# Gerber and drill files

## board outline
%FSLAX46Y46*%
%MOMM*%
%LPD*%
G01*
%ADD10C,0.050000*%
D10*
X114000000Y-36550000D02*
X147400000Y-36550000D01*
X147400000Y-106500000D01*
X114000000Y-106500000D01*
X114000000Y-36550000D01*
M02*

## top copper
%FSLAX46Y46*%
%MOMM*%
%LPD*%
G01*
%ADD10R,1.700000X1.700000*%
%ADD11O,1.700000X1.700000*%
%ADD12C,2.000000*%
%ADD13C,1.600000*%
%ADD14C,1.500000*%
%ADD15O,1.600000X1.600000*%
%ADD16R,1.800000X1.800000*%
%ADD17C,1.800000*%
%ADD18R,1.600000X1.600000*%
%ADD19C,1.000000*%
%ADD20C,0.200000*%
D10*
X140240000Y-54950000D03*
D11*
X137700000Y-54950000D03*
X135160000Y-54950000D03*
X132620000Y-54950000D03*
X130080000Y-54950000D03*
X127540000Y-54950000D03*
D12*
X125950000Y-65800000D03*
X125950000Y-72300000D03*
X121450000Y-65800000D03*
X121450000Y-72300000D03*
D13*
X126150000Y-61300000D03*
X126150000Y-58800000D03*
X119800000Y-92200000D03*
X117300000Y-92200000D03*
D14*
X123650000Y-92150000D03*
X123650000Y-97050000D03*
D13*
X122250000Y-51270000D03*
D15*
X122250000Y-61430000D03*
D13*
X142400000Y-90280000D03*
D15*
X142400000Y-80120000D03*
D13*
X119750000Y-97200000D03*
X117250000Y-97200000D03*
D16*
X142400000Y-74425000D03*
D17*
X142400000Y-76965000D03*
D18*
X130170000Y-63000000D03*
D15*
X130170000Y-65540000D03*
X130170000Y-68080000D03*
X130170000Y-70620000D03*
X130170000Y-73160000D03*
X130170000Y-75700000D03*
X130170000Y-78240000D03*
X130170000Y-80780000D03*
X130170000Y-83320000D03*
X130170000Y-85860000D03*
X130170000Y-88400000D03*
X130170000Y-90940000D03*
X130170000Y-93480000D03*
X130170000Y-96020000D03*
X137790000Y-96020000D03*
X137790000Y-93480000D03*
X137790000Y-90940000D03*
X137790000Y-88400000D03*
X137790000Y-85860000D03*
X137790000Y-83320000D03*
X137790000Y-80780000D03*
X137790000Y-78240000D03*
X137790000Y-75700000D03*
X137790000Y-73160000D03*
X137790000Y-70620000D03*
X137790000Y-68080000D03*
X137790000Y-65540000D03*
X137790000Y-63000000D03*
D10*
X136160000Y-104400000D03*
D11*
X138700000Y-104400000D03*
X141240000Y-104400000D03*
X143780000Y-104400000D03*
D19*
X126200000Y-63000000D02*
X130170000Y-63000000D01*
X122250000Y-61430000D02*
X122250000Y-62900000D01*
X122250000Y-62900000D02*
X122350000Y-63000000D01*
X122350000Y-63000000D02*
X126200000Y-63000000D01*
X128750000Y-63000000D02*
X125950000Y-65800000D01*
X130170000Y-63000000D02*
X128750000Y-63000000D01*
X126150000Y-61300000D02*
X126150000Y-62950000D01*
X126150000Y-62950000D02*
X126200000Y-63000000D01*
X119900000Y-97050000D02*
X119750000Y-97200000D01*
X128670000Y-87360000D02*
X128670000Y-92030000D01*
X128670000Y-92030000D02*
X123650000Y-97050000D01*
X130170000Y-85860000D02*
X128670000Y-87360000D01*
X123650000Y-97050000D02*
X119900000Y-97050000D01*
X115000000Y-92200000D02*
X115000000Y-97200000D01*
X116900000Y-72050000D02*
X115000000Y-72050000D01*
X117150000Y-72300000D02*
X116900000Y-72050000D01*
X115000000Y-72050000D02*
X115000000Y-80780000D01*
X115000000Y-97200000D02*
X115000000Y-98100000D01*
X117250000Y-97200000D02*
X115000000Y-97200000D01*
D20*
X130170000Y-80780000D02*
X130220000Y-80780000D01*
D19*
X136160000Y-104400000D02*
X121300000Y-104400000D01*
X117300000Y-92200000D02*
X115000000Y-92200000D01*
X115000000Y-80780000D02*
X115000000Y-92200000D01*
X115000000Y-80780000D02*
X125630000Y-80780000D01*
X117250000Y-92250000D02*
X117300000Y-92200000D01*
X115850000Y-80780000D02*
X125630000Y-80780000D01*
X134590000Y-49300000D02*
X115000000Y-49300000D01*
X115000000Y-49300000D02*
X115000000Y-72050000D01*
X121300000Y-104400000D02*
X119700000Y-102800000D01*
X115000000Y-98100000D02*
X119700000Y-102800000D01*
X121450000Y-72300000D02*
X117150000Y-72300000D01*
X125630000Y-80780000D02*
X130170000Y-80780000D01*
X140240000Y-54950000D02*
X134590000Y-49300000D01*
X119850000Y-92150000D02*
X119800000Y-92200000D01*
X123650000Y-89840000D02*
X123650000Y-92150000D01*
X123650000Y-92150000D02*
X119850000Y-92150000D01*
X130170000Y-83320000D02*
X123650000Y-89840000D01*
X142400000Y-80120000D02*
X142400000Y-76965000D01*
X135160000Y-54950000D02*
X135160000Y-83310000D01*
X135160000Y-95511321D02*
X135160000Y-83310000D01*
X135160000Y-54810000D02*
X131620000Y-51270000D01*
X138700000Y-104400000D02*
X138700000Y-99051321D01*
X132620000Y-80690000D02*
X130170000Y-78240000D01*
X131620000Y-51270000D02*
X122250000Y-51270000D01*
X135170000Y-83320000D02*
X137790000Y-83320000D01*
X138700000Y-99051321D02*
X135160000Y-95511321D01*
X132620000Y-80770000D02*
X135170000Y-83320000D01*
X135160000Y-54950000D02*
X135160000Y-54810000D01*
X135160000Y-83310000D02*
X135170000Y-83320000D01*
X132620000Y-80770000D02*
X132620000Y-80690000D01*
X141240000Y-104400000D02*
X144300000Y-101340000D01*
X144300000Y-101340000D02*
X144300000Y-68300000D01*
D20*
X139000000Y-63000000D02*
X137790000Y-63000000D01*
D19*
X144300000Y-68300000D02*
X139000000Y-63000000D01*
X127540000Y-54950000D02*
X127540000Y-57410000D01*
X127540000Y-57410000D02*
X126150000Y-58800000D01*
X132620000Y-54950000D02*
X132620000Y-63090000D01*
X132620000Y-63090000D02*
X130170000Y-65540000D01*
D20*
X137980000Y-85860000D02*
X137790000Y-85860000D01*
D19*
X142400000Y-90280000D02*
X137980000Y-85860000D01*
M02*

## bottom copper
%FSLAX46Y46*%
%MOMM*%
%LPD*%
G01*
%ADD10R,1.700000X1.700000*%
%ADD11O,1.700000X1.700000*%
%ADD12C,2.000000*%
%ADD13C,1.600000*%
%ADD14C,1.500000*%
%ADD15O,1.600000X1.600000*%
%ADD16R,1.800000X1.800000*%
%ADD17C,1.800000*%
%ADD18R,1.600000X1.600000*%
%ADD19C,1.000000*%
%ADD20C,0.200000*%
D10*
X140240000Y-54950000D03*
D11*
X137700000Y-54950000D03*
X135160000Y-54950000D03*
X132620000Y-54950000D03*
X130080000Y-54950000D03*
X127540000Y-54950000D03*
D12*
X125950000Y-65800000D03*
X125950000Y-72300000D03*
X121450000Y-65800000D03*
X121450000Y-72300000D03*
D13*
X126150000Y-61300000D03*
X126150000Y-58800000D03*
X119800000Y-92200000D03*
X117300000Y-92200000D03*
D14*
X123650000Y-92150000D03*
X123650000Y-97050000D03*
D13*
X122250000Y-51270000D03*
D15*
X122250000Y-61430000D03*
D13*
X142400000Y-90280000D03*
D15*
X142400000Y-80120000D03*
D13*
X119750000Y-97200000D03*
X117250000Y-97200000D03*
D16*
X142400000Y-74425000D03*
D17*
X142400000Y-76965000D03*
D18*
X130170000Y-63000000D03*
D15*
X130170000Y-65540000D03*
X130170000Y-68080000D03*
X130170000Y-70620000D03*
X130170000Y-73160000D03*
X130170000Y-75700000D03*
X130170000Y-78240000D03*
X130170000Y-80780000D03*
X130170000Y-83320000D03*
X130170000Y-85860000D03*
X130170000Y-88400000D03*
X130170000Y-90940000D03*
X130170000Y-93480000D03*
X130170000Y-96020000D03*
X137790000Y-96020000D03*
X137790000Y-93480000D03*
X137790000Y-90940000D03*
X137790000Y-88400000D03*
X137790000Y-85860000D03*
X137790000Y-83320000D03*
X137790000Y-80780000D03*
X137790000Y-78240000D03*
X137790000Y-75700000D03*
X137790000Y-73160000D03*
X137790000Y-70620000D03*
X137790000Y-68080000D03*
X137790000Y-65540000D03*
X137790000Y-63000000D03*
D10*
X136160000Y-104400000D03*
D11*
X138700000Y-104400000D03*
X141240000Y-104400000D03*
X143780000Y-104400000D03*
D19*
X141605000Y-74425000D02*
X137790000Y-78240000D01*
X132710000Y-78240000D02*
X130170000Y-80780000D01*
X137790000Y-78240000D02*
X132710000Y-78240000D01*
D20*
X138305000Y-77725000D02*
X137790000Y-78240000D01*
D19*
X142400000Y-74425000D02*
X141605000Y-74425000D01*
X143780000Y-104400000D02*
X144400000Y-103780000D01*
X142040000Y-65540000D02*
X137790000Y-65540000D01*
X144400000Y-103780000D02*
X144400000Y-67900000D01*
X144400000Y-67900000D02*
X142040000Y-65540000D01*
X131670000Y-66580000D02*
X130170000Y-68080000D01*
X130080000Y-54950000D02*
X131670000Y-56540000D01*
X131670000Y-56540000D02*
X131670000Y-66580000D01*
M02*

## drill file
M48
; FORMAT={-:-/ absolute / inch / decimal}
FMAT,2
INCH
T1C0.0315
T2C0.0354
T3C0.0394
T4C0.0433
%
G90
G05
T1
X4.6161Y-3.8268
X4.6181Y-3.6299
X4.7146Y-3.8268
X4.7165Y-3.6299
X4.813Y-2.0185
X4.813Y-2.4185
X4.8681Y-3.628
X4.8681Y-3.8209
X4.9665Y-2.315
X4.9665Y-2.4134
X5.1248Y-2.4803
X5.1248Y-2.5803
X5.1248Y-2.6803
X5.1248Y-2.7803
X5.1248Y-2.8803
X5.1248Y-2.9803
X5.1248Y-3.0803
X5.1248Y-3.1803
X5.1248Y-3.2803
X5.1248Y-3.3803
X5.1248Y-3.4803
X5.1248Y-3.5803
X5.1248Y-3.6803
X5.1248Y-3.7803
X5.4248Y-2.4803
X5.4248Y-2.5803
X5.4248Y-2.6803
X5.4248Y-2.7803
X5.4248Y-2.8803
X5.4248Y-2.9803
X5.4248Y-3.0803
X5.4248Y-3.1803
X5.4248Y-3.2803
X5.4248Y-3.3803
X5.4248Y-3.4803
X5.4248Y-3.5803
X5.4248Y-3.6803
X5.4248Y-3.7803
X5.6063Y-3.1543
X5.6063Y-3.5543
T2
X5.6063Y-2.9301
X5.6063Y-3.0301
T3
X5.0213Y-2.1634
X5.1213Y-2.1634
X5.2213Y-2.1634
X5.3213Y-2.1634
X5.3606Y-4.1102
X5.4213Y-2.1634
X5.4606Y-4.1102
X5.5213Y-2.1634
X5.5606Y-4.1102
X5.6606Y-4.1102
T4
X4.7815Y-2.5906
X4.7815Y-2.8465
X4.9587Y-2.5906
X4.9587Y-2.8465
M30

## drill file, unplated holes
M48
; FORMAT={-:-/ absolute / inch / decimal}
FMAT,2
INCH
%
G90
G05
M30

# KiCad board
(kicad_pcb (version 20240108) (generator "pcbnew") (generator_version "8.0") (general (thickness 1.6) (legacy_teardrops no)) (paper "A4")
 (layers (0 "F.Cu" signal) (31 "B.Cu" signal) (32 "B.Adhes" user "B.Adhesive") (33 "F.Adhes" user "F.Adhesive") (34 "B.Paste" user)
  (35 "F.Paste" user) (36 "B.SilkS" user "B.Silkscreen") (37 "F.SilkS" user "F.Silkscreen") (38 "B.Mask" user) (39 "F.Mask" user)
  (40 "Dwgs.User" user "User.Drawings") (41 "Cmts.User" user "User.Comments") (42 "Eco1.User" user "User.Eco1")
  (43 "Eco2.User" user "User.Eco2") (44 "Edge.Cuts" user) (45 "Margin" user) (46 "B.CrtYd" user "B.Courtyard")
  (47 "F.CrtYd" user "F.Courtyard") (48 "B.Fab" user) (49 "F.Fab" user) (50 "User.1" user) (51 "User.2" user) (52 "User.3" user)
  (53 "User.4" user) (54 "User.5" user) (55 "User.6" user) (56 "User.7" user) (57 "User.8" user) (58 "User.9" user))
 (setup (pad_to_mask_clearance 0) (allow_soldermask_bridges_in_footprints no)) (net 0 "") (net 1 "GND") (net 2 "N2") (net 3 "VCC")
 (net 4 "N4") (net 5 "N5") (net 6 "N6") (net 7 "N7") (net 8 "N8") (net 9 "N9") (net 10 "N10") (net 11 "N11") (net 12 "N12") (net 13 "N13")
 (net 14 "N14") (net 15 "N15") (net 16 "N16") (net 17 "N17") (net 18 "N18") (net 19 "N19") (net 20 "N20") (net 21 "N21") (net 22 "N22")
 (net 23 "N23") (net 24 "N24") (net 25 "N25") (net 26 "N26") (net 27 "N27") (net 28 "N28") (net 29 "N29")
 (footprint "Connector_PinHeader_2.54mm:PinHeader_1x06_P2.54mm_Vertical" (layer "F.Cu") (at 140.24 54.95 -90)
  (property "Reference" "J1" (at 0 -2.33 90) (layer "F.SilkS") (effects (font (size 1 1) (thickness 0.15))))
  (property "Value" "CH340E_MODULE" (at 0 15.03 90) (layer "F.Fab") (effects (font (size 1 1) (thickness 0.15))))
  (pad "1" thru_hole rect (at 0 0 270) (size 1.7 1.7) (drill 1) (layers "*.Cu" "*.Mask") (remove_unused_layers no) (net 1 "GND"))
  (pad "2" thru_hole oval (at 0 2.54 270) (size 1.7 1.7) (drill 1) (layers "*.Cu" "*.Mask") (remove_unused_layers no) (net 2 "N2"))
  (pad "3" thru_hole oval (at 0 5.08 270) (size 1.7 1.7) (drill 1) (layers "*.Cu" "*.Mask") (remove_unused_layers no) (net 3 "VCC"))
  (pad "4" thru_hole oval (at 0 7.62 270) (size 1.7 1.7) (drill 1) (layers "*.Cu" "*.Mask") (remove_unused_layers no) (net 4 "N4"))
  (pad "5" thru_hole oval (at 0 10.16 270) (size 1.7 1.7) (drill 1) (layers "*.Cu" "*.Mask") (remove_unused_layers no) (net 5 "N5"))
  (pad "6" thru_hole oval (at 0 12.7 270) (size 1.7 1.7) (drill 1) (layers "*.Cu" "*.Mask") (remove_unused_layers no) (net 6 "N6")))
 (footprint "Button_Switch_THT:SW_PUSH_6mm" (layer "F.Cu") (at 125.95 65.8 -90)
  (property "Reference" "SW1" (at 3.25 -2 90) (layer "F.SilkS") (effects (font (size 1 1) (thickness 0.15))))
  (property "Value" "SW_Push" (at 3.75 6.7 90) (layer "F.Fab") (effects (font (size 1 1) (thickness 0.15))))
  (pad "1" thru_hole circle (at 0 0) (size 2 2) (drill 1.1) (layers "*.Cu" "*.Mask") (remove_unused_layers no) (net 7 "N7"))
  (pad "1" thru_hole circle (at 6.5 0) (size 2 2) (drill 1.1) (layers "*.Cu" "*.Mask") (remove_unused_layers no) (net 7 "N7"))
  (pad "2" thru_hole circle (at 0 4.5) (size 2 2) (drill 1.1) (layers "*.Cu" "*.Mask") (remove_unused_layers no) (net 1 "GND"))
  (pad "2" thru_hole circle (at 6.5 4.5) (size 2 2) (drill 1.1) (layers "*.Cu" "*.Mask") (remove_unused_layers no) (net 1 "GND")))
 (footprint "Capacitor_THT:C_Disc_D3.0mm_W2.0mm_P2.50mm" (layer "F.Cu") (at 126.15 61.3 90)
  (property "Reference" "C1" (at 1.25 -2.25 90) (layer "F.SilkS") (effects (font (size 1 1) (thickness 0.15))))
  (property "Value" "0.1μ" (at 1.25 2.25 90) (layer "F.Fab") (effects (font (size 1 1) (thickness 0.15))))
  (pad "1" thru_hole circle (at 0 0 90) (size 1.6 1.6) (drill 0.8) (layers "*.Cu" "*.Mask") (remove_unused_layers no) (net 7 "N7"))
  (pad "2" thru_hole circle (at 2.5 0 90) (size 1.6 1.6) (drill 0.8) (layers "*.Cu" "*.Mask") (remove_unused_layers no) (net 6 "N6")))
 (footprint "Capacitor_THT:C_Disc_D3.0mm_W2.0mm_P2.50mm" (layer "F.Cu") (at 119.8 92.2 180)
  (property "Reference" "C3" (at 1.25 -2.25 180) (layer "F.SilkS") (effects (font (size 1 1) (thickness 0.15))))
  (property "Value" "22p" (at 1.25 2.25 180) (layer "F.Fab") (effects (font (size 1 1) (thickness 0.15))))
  (pad "1" thru_hole circle (at 0 0 180) (size 1.6 1.6) (drill 0.8) (layers "*.Cu" "*.Mask") (remove_unused_layers no) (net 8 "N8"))
  (pad "2" thru_hole circle (at 2.5 0 180) (size 1.6 1.6) (drill 0.8) (layers "*.Cu" "*.Mask") (remove_unused_layers no) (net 1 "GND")))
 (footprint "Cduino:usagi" (layer "F.Cu") (at 137.448475 45.277091)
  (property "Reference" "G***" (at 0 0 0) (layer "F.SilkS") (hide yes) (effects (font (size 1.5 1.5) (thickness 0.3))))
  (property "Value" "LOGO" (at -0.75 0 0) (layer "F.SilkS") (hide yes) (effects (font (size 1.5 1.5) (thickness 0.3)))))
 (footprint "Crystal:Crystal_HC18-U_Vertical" (layer "F.Cu") (at 123.65 92.15 -90)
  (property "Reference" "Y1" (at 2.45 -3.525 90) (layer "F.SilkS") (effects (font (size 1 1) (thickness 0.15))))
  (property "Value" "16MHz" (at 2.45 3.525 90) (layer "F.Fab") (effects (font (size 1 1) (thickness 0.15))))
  (pad "1" thru_hole circle (at 0 0 270) (size 1.5 1.5) (drill 0.8) (layers "*.Cu" "*.Mask") (remove_unused_layers no) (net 8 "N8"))
  (pad "2" thru_hole circle (at 4.9 0 270) (size 1.5 1.5) (drill 0.8) (layers "*.Cu" "*.Mask") (remove_unused_layers no) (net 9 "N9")))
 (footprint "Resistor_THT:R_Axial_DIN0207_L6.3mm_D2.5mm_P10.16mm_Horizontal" (layer "F.Cu") (at 122.25 51.27 -90)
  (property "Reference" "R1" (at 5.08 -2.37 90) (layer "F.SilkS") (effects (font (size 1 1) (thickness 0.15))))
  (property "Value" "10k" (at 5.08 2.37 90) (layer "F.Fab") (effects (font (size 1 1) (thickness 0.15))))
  (pad "1" thru_hole circle (at 0 0 270) (size 1.6 1.6) (drill 0.8) (layers "*.Cu" "*.Mask") (remove_unused_layers no) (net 3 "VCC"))
  (pad "2" thru_hole oval (at 10.16 0 270) (size 1.6 1.6) (drill 0.8) (layers "*.Cu" "*.Mask") (remove_unused_layers no) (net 7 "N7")))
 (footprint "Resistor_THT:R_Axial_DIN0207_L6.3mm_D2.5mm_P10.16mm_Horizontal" (layer "F.Cu") (at 142.4 90.28 90)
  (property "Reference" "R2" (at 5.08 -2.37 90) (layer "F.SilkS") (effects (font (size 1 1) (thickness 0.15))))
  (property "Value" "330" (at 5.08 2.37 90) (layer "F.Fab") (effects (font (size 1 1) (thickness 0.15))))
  (pad "1" thru_hole circle (at 0 0 90) (size 1.6 1.6) (drill 0.8) (layers "*.Cu" "*.Mask") (remove_unused_layers no) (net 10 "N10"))
  (pad "2" thru_hole oval (at 10.16 0 90) (size 1.6 1.6) (drill 0.8) (layers "*.Cu" "*.Mask") (remove_unused_layers no) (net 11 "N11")))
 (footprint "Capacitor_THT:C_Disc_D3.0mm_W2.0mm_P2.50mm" (layer "F.Cu") (at 119.75 97.2 180)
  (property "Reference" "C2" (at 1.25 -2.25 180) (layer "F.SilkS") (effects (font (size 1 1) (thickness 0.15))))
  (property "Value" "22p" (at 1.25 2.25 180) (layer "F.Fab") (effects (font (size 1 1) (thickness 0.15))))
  (pad "1" thru_hole circle (at 0 0 180) (size 1.6 1.6) (drill 0.8) (layers "*.Cu" "*.Mask") (remove_unused_layers no) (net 9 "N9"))
  (pad "2" thru_hole circle (at 2.5 0 180) (size 1.6 1.6) (drill 0.8) (layers "*.Cu" "*.Mask") (remove_unused_layers no) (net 1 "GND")))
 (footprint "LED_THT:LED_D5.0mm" (layer "F.Cu") (at 142.4 74.425 -90)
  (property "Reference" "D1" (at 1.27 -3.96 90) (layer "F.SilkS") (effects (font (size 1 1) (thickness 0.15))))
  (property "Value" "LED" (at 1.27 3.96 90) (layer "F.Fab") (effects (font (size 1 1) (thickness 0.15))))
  (pad "1" thru_hole rect (at 0 0 270) (size 1.8 1.8) (drill 0.9) (layers "*.Cu" "*.Mask") (remove_unused_layers no) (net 1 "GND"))
  (pad "2" thru_hole circle (at 2.54 0 270) (size 1.8 1.8) (drill 0.9) (layers "*.Cu" "*.Mask") (remove_unused_layers no) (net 11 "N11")))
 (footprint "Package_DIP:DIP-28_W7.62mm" (layer "F.Cu") (at 130.17 63)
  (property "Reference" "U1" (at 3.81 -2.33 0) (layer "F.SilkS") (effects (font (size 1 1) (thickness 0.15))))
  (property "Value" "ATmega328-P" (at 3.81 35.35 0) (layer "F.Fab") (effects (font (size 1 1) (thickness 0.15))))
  (pad "1" thru_hole rect (at 0 0) (size 1.6 1.6) (drill 0.8) (layers "*.Cu" "*.Mask") (remove_unused_layers no) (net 7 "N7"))
  (pad "2" thru_hole oval (at 0 2.54) (size 1.6 1.6) (drill 0.8) (layers "*.Cu" "*.Mask") (remove_unused_layers no) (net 4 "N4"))
  (pad "3" thru_hole oval (at 0 5.08) (size 1.6 1.6) (drill 0.8) (layers "*.Cu" "*.Mask") (remove_unused_layers no) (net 5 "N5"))
  (pad "4" thru_hole oval (at 0 7.62) (size 1.6 1.6) (drill 0.8) (layers "*.Cu" "*.Mask") (remove_unused_layers no) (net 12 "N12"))
  (pad "5" thru_hole oval (at 0 10.16) (size 1.6 1.6) (drill 0.8) (layers "*.Cu" "*.Mask") (remove_unused_layers no) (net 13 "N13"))
  (pad "6" thru_hole oval (at 0 12.7) (size 1.6 1.6) (drill 0.8) (layers "*.Cu" "*.Mask") (remove_unused_layers no) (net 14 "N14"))
  (pad "7" thru_hole oval (at 0 15.24) (size 1.6 1.6) (drill 0.8) (layers "*.Cu" "*.Mask") (remove_unused_layers no) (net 3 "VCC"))
  (pad "8" thru_hole oval (at 0 17.78) (size 1.6 1.6) (drill 0.8) (layers "*.Cu" "*.Mask") (remove_unused_layers no) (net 1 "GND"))
  (pad "9" thru_hole oval (at 0 20.32) (size 1.6 1.6) (drill 0.8) (layers "*.Cu" "*.Mask") (remove_unused_layers no) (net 8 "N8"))
  (pad "10" thru_hole oval (at 0 22.86) (size 1.6 1.6) (drill 0.8) (layers "*.Cu" "*.Mask") (remove_unused_layers no) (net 9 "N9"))
  (pad "11" thru_hole oval (at 0 25.4) (size 1.6 1.6) (drill 0.8) (layers "*.Cu" "*.Mask") (remove_unused_layers no) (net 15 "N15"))
  (pad "12" thru_hole oval (at 0 27.94) (size 1.6 1.6) (drill 0.8) (layers "*.Cu" "*.Mask") (remove_unused_layers no) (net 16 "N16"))
  (pad "13" thru_hole oval (at 0 30.48) (size 1.6 1.6) (drill 0.8) (layers "*.Cu" "*.Mask") (remove_unused_layers no) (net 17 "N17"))
  (pad "14" thru_hole oval (at 0 33.02) (size 1.6 1.6) (drill 0.8) (layers "*.Cu" "*.Mask") (remove_unused_layers no) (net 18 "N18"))
  (pad "15" thru_hole oval (at 7.62 33.02) (size 1.6 1.6) (drill 0.8) (layers "*.Cu" "*.Mask") (remove_unused_layers no) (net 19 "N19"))
  (pad "16" thru_hole oval (at 7.62 30.48) (size 1.6 1.6) (drill 0.8) (layers "*.Cu" "*.Mask") (remove_unused_layers no) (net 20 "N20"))
  (pad "17" thru_hole oval (at 7.62 27.94) (size 1.6 1.6) (drill 0.8) (layers "*.Cu" "*.Mask") (remove_unused_layers no) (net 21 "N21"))
  (pad "18" thru_hole oval (at 7.62 25.4) (size 1.6 1.6) (drill 0.8) (layers "*.Cu" "*.Mask") (remove_unused_layers no) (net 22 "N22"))
  (pad "19" thru_hole oval (at 7.62 22.86) (size 1.6 1.6) (drill 0.8) (layers "*.Cu" "*.Mask") (remove_unused_layers no) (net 10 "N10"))
  (pad "20" thru_hole oval (at 7.62 20.32) (size 1.6 1.6) (drill 0.8) (layers "*.Cu" "*.Mask") (remove_unused_layers no) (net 3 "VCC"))
  (pad "21" thru_hole oval (at 7.62 17.78) (size 1.6 1.6) (drill 0.8) (layers "*.Cu" "*.Mask") (remove_unused_layers no) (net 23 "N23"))
  (pad "22" thru_hole oval (at 7.62 15.24) (size 1.6 1.6) (drill 0.8) (layers "*.Cu" "*.Mask") (remove_unused_layers no) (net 1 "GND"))
  (pad "23" thru_hole oval (at 7.62 12.7) (size 1.6 1.6) (drill 0.8) (layers "*.Cu" "*.Mask") (remove_unused_layers no) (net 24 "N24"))
  (pad "24" thru_hole oval (at 7.62 10.16) (size 1.6 1.6) (drill 0.8) (layers "*.Cu" "*.Mask") (remove_unused_layers no) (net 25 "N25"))
  (pad "25" thru_hole oval (at 7.62 7.62) (size 1.6 1.6) (drill 0.8) (layers "*.Cu" "*.Mask") (remove_unused_layers no) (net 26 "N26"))
  (pad "26" thru_hole oval (at 7.62 5.08) (size 1.6 1.6) (drill 0.8) (layers "*.Cu" "*.Mask") (remove_unused_layers no) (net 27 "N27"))
  (pad "27" thru_hole oval (at 7.62 2.54) (size 1.6 1.6) (drill 0.8) (layers "*.Cu" "*.Mask") (remove_unused_layers no) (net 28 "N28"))
  (pad "28" thru_hole oval (at 7.62 0) (size 1.6 1.6) (drill 0.8) (layers "*.Cu" "*.Mask") (remove_unused_layers no) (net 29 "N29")))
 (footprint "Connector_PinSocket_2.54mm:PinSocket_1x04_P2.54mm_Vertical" (layer "F.Cu") (at 136.16 104.4 90)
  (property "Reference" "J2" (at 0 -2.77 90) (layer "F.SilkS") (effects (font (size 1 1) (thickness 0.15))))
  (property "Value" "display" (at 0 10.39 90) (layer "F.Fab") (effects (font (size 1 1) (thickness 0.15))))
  (pad "1" thru_hole rect (at 0 0 90) (size 1.7 1.7) (drill 1) (layers "*.Cu" "*.Mask") (remove_unused_layers no) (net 1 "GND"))
  (pad "2" thru_hole oval (at 0 2.54 90) (size 1.7 1.7) (drill 1) (layers "*.Cu" "*.Mask") (remove_unused_layers no) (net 3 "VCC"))
  (pad "3" thru_hole oval (at 0 5.08 90) (size 1.7 1.7) (drill 1) (layers "*.Cu" "*.Mask") (remove_unused_layers no) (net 29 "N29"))
  (pad "4" thru_hole oval (at 0 7.62 90) (size 1.7 1.7) (drill 1) (layers "*.Cu" "*.Mask") (remove_unused_layers no) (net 28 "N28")))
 (gr_rect (start 114 36.55) (end 147.4 106.5) (stroke (width 0.05) (type default)) (fill none) (layer "Edge.Cuts"))
 (segment (start 126.2 63) (end 130.17 63) (width 1) (layer "F.Cu") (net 7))
 (segment (start 122.25 61.43) (end 122.25 62.9) (width 1) (layer "F.Cu") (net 7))
 (segment (start 122.25 62.9) (end 122.35 63) (width 1) (layer "F.Cu") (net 7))
 (segment (start 122.35 63) (end 126.2 63) (width 1) (layer "F.Cu") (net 7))
 (segment (start 128.75 63) (end 125.95 65.8) (width 1) (layer "F.Cu") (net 7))
 (segment (start 130.17 63) (end 128.75 63) (width 1) (layer "F.Cu") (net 7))
 (segment (start 126.15 61.3) (end 126.15 62.95) (width 1) (layer "F.Cu") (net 7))
 (segment (start 126.15 62.95) (end 126.2 63) (width 1) (layer "F.Cu") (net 7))
 (segment (start 119.9 97.05) (end 119.75 97.2) (width 1) (layer "F.Cu") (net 9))
 (segment (start 128.67 87.36) (end 128.67 92.03) (width 1) (layer "F.Cu") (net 9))
 (segment (start 128.67 92.03) (end 123.65 97.05) (width 1) (layer "F.Cu") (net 9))
 (segment (start 130.17 85.86) (end 128.67 87.36) (width 1) (layer "F.Cu") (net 9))
 (segment (start 123.65 97.05) (end 119.9 97.05) (width 1) (layer "F.Cu") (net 9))
 (segment (start 115 92.2) (end 115 97.2) (width 1) (layer "F.Cu") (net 1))
 (segment (start 116.9 72.05) (end 115 72.05) (width 1) (layer "F.Cu") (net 1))
 (segment (start 117.15 72.3) (end 116.9 72.05) (width 1) (layer "F.Cu") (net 1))
 (segment (start 115 72.05) (end 115 80.78) (width 1) (layer "F.Cu") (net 1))
 (segment (start 115 97.2) (end 115 98.1) (width 1) (layer "F.Cu") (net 1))
 (segment (start 117.25 97.2) (end 115 97.2) (width 1) (layer "F.Cu") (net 1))
 (segment (start 130.17 80.78) (end 130.22 80.78) (width 0.2) (layer "F.Cu") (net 1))
 (segment (start 136.16 104.4) (end 121.3 104.4) (width 1) (layer "F.Cu") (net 1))
 (segment (start 117.3 92.2) (end 115 92.2) (width 1) (layer "F.Cu") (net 1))
 (segment (start 115 80.78) (end 115 92.2) (width 1) (layer "F.Cu") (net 1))
 (segment (start 115 80.78) (end 125.63 80.78) (width 1) (layer "F.Cu") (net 1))
 (segment (start 117.25 92.25) (end 117.3 92.2) (width 1) (layer "F.Cu") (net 1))
 (segment (start 115.85 80.78) (end 125.63 80.78) (width 1) (layer "F.Cu") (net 1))
 (segment (start 134.59 49.3) (end 115 49.3) (width 1) (layer "F.Cu") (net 1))
 (segment (start 115 49.3) (end 115 72.05) (width 1) (layer "F.Cu") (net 1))
 (segment (start 121.3 104.4) (end 119.7 102.8) (width 1) (layer "F.Cu") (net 1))
 (segment (start 115 98.1) (end 119.7 102.8) (width 1) (layer "F.Cu") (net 1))
 (segment (start 121.45 72.3) (end 117.15 72.3) (width 1) (layer "F.Cu") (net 1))
 (segment (start 125.63 80.78) (end 130.17 80.78) (width 1) (layer "F.Cu") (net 1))
 (segment (start 140.24 54.95) (end 134.59 49.3) (width 1) (layer "F.Cu") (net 1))
 (segment (start 141.605 74.425) (end 137.79 78.24) (width 1) (layer "B.Cu") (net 1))
 (segment (start 132.71 78.24) (end 130.17 80.78) (width 1) (layer "B.Cu") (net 1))
 (segment (start 137.79 78.24) (end 132.71 78.24) (width 1) (layer "B.Cu") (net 1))
 (segment (start 138.305 77.725) (end 137.79 78.24) (width 0.2) (layer "B.Cu") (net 1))
 (segment (start 142.4 74.425) (end 141.605 74.425) (width 1) (layer "B.Cu") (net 1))
 (segment (start 119.85 92.15) (end 119.8 92.2) (width 1) (layer "F.Cu") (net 8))
 (segment (start 123.65 89.84) (end 123.65 92.15) (width 1) (layer "F.Cu") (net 8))
 (segment (start 123.65 92.15) (end 119.85 92.15) (width 1) (layer "F.Cu") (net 8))
 (segment (start 130.17 83.32) (end 123.65 89.84) (width 1) (layer "F.Cu") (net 8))
 (segment (start 142.4 80.12) (end 142.4 76.965) (width 1) (layer "F.Cu") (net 11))
 (segment (start 135.16 54.95) (end 135.16 83.31) (width 1) (layer "F.Cu") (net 3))
 (segment (start 135.16 95.511321) (end 135.16 83.31) (width 1) (layer "F.Cu") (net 3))
 (segment (start 135.16 54.81) (end 131.62 51.27) (width 1) (layer "F.Cu") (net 3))
 (segment (start 138.7 104.4) (end 138.7 99.051321) (width 1) (layer "F.Cu") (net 3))
 (segment (start 132.62 80.69) (end 130.17 78.24) (width 1) (layer "F.Cu") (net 3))
 (segment (start 131.62 51.27) (end 122.25 51.27) (width 1) (layer "F.Cu") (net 3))
 (segment (start 135.17 83.32) (end 137.79 83.32) (width 1) (layer "F.Cu") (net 3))
 (segment (start 138.7 99.051321) (end 135.16 95.511321) (width 1) (layer "F.Cu") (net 3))
 (segment (start 132.62 80.77) (end 135.17 83.32) (width 1) (layer "F.Cu") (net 3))
 (segment (start 135.16 54.95) (end 135.16 54.81) (width 1) (layer "F.Cu") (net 3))
 (segment (start 135.16 83.31) (end 135.17 83.32) (width 1) (layer "F.Cu") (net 3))
 (segment (start 132.62 80.77) (end 132.62 80.69) (width 1) (layer "F.Cu") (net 3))
 (segment (start 141.24 104.4) (end 144.3 101.34) (width 1) (layer "F.Cu") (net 29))
 (segment (start 144.3 101.34) (end 144.3 68.3) (width 1) (layer "F.Cu") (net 29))
 (segment (start 139 63) (end 137.79 63) (width 0.2) (layer "F.Cu") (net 29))
 (segment (start 144.3 68.3) (end 139 63) (width 1) (layer "F.Cu") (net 29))
 (segment (start 143.78 104.4) (end 144.4 103.78) (width 1) (layer "B.Cu") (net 28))
 (segment (start 142.04 65.54) (end 137.79 65.54) (width 1) (layer "B.Cu") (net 28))
 (segment (start 144.4 103.78) (end 144.4 67.9) (width 1) (layer "B.Cu") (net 28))
 (segment (start 144.4 67.9) (end 142.04 65.54) (width 1) (layer "B.Cu") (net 28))
 (segment (start 127.54 54.95) (end 127.54 57.41) (width 1) (layer "F.Cu") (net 6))
 (segment (start 127.54 57.41) (end 126.15 58.8) (width 1) (layer "F.Cu") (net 6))
 (segment (start 131.67 66.58) (end 130.17 68.08) (width 1) (layer "B.Cu") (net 5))
 (segment (start 130.08 54.95) (end 131.67 56.54) (width 1) (layer "B.Cu") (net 5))
 (segment (start 131.67 56.54) (end 131.67 66.58) (width 1) (layer "B.Cu") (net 5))
 (segment (start 132.62 54.95) (end 132.62 63.09) (width 1) (layer "F.Cu") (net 4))
 (segment (start 132.62 63.09) (end 130.17 65.54) (width 1) (layer "F.Cu") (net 4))
 (segment (start 137.98 85.86) (end 137.79 85.86) (width 0.2) (layer "F.Cu") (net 10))
 (segment (start 142.4 90.28) (end 137.98 85.86) (width 1) (layer "F.Cu") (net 10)))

